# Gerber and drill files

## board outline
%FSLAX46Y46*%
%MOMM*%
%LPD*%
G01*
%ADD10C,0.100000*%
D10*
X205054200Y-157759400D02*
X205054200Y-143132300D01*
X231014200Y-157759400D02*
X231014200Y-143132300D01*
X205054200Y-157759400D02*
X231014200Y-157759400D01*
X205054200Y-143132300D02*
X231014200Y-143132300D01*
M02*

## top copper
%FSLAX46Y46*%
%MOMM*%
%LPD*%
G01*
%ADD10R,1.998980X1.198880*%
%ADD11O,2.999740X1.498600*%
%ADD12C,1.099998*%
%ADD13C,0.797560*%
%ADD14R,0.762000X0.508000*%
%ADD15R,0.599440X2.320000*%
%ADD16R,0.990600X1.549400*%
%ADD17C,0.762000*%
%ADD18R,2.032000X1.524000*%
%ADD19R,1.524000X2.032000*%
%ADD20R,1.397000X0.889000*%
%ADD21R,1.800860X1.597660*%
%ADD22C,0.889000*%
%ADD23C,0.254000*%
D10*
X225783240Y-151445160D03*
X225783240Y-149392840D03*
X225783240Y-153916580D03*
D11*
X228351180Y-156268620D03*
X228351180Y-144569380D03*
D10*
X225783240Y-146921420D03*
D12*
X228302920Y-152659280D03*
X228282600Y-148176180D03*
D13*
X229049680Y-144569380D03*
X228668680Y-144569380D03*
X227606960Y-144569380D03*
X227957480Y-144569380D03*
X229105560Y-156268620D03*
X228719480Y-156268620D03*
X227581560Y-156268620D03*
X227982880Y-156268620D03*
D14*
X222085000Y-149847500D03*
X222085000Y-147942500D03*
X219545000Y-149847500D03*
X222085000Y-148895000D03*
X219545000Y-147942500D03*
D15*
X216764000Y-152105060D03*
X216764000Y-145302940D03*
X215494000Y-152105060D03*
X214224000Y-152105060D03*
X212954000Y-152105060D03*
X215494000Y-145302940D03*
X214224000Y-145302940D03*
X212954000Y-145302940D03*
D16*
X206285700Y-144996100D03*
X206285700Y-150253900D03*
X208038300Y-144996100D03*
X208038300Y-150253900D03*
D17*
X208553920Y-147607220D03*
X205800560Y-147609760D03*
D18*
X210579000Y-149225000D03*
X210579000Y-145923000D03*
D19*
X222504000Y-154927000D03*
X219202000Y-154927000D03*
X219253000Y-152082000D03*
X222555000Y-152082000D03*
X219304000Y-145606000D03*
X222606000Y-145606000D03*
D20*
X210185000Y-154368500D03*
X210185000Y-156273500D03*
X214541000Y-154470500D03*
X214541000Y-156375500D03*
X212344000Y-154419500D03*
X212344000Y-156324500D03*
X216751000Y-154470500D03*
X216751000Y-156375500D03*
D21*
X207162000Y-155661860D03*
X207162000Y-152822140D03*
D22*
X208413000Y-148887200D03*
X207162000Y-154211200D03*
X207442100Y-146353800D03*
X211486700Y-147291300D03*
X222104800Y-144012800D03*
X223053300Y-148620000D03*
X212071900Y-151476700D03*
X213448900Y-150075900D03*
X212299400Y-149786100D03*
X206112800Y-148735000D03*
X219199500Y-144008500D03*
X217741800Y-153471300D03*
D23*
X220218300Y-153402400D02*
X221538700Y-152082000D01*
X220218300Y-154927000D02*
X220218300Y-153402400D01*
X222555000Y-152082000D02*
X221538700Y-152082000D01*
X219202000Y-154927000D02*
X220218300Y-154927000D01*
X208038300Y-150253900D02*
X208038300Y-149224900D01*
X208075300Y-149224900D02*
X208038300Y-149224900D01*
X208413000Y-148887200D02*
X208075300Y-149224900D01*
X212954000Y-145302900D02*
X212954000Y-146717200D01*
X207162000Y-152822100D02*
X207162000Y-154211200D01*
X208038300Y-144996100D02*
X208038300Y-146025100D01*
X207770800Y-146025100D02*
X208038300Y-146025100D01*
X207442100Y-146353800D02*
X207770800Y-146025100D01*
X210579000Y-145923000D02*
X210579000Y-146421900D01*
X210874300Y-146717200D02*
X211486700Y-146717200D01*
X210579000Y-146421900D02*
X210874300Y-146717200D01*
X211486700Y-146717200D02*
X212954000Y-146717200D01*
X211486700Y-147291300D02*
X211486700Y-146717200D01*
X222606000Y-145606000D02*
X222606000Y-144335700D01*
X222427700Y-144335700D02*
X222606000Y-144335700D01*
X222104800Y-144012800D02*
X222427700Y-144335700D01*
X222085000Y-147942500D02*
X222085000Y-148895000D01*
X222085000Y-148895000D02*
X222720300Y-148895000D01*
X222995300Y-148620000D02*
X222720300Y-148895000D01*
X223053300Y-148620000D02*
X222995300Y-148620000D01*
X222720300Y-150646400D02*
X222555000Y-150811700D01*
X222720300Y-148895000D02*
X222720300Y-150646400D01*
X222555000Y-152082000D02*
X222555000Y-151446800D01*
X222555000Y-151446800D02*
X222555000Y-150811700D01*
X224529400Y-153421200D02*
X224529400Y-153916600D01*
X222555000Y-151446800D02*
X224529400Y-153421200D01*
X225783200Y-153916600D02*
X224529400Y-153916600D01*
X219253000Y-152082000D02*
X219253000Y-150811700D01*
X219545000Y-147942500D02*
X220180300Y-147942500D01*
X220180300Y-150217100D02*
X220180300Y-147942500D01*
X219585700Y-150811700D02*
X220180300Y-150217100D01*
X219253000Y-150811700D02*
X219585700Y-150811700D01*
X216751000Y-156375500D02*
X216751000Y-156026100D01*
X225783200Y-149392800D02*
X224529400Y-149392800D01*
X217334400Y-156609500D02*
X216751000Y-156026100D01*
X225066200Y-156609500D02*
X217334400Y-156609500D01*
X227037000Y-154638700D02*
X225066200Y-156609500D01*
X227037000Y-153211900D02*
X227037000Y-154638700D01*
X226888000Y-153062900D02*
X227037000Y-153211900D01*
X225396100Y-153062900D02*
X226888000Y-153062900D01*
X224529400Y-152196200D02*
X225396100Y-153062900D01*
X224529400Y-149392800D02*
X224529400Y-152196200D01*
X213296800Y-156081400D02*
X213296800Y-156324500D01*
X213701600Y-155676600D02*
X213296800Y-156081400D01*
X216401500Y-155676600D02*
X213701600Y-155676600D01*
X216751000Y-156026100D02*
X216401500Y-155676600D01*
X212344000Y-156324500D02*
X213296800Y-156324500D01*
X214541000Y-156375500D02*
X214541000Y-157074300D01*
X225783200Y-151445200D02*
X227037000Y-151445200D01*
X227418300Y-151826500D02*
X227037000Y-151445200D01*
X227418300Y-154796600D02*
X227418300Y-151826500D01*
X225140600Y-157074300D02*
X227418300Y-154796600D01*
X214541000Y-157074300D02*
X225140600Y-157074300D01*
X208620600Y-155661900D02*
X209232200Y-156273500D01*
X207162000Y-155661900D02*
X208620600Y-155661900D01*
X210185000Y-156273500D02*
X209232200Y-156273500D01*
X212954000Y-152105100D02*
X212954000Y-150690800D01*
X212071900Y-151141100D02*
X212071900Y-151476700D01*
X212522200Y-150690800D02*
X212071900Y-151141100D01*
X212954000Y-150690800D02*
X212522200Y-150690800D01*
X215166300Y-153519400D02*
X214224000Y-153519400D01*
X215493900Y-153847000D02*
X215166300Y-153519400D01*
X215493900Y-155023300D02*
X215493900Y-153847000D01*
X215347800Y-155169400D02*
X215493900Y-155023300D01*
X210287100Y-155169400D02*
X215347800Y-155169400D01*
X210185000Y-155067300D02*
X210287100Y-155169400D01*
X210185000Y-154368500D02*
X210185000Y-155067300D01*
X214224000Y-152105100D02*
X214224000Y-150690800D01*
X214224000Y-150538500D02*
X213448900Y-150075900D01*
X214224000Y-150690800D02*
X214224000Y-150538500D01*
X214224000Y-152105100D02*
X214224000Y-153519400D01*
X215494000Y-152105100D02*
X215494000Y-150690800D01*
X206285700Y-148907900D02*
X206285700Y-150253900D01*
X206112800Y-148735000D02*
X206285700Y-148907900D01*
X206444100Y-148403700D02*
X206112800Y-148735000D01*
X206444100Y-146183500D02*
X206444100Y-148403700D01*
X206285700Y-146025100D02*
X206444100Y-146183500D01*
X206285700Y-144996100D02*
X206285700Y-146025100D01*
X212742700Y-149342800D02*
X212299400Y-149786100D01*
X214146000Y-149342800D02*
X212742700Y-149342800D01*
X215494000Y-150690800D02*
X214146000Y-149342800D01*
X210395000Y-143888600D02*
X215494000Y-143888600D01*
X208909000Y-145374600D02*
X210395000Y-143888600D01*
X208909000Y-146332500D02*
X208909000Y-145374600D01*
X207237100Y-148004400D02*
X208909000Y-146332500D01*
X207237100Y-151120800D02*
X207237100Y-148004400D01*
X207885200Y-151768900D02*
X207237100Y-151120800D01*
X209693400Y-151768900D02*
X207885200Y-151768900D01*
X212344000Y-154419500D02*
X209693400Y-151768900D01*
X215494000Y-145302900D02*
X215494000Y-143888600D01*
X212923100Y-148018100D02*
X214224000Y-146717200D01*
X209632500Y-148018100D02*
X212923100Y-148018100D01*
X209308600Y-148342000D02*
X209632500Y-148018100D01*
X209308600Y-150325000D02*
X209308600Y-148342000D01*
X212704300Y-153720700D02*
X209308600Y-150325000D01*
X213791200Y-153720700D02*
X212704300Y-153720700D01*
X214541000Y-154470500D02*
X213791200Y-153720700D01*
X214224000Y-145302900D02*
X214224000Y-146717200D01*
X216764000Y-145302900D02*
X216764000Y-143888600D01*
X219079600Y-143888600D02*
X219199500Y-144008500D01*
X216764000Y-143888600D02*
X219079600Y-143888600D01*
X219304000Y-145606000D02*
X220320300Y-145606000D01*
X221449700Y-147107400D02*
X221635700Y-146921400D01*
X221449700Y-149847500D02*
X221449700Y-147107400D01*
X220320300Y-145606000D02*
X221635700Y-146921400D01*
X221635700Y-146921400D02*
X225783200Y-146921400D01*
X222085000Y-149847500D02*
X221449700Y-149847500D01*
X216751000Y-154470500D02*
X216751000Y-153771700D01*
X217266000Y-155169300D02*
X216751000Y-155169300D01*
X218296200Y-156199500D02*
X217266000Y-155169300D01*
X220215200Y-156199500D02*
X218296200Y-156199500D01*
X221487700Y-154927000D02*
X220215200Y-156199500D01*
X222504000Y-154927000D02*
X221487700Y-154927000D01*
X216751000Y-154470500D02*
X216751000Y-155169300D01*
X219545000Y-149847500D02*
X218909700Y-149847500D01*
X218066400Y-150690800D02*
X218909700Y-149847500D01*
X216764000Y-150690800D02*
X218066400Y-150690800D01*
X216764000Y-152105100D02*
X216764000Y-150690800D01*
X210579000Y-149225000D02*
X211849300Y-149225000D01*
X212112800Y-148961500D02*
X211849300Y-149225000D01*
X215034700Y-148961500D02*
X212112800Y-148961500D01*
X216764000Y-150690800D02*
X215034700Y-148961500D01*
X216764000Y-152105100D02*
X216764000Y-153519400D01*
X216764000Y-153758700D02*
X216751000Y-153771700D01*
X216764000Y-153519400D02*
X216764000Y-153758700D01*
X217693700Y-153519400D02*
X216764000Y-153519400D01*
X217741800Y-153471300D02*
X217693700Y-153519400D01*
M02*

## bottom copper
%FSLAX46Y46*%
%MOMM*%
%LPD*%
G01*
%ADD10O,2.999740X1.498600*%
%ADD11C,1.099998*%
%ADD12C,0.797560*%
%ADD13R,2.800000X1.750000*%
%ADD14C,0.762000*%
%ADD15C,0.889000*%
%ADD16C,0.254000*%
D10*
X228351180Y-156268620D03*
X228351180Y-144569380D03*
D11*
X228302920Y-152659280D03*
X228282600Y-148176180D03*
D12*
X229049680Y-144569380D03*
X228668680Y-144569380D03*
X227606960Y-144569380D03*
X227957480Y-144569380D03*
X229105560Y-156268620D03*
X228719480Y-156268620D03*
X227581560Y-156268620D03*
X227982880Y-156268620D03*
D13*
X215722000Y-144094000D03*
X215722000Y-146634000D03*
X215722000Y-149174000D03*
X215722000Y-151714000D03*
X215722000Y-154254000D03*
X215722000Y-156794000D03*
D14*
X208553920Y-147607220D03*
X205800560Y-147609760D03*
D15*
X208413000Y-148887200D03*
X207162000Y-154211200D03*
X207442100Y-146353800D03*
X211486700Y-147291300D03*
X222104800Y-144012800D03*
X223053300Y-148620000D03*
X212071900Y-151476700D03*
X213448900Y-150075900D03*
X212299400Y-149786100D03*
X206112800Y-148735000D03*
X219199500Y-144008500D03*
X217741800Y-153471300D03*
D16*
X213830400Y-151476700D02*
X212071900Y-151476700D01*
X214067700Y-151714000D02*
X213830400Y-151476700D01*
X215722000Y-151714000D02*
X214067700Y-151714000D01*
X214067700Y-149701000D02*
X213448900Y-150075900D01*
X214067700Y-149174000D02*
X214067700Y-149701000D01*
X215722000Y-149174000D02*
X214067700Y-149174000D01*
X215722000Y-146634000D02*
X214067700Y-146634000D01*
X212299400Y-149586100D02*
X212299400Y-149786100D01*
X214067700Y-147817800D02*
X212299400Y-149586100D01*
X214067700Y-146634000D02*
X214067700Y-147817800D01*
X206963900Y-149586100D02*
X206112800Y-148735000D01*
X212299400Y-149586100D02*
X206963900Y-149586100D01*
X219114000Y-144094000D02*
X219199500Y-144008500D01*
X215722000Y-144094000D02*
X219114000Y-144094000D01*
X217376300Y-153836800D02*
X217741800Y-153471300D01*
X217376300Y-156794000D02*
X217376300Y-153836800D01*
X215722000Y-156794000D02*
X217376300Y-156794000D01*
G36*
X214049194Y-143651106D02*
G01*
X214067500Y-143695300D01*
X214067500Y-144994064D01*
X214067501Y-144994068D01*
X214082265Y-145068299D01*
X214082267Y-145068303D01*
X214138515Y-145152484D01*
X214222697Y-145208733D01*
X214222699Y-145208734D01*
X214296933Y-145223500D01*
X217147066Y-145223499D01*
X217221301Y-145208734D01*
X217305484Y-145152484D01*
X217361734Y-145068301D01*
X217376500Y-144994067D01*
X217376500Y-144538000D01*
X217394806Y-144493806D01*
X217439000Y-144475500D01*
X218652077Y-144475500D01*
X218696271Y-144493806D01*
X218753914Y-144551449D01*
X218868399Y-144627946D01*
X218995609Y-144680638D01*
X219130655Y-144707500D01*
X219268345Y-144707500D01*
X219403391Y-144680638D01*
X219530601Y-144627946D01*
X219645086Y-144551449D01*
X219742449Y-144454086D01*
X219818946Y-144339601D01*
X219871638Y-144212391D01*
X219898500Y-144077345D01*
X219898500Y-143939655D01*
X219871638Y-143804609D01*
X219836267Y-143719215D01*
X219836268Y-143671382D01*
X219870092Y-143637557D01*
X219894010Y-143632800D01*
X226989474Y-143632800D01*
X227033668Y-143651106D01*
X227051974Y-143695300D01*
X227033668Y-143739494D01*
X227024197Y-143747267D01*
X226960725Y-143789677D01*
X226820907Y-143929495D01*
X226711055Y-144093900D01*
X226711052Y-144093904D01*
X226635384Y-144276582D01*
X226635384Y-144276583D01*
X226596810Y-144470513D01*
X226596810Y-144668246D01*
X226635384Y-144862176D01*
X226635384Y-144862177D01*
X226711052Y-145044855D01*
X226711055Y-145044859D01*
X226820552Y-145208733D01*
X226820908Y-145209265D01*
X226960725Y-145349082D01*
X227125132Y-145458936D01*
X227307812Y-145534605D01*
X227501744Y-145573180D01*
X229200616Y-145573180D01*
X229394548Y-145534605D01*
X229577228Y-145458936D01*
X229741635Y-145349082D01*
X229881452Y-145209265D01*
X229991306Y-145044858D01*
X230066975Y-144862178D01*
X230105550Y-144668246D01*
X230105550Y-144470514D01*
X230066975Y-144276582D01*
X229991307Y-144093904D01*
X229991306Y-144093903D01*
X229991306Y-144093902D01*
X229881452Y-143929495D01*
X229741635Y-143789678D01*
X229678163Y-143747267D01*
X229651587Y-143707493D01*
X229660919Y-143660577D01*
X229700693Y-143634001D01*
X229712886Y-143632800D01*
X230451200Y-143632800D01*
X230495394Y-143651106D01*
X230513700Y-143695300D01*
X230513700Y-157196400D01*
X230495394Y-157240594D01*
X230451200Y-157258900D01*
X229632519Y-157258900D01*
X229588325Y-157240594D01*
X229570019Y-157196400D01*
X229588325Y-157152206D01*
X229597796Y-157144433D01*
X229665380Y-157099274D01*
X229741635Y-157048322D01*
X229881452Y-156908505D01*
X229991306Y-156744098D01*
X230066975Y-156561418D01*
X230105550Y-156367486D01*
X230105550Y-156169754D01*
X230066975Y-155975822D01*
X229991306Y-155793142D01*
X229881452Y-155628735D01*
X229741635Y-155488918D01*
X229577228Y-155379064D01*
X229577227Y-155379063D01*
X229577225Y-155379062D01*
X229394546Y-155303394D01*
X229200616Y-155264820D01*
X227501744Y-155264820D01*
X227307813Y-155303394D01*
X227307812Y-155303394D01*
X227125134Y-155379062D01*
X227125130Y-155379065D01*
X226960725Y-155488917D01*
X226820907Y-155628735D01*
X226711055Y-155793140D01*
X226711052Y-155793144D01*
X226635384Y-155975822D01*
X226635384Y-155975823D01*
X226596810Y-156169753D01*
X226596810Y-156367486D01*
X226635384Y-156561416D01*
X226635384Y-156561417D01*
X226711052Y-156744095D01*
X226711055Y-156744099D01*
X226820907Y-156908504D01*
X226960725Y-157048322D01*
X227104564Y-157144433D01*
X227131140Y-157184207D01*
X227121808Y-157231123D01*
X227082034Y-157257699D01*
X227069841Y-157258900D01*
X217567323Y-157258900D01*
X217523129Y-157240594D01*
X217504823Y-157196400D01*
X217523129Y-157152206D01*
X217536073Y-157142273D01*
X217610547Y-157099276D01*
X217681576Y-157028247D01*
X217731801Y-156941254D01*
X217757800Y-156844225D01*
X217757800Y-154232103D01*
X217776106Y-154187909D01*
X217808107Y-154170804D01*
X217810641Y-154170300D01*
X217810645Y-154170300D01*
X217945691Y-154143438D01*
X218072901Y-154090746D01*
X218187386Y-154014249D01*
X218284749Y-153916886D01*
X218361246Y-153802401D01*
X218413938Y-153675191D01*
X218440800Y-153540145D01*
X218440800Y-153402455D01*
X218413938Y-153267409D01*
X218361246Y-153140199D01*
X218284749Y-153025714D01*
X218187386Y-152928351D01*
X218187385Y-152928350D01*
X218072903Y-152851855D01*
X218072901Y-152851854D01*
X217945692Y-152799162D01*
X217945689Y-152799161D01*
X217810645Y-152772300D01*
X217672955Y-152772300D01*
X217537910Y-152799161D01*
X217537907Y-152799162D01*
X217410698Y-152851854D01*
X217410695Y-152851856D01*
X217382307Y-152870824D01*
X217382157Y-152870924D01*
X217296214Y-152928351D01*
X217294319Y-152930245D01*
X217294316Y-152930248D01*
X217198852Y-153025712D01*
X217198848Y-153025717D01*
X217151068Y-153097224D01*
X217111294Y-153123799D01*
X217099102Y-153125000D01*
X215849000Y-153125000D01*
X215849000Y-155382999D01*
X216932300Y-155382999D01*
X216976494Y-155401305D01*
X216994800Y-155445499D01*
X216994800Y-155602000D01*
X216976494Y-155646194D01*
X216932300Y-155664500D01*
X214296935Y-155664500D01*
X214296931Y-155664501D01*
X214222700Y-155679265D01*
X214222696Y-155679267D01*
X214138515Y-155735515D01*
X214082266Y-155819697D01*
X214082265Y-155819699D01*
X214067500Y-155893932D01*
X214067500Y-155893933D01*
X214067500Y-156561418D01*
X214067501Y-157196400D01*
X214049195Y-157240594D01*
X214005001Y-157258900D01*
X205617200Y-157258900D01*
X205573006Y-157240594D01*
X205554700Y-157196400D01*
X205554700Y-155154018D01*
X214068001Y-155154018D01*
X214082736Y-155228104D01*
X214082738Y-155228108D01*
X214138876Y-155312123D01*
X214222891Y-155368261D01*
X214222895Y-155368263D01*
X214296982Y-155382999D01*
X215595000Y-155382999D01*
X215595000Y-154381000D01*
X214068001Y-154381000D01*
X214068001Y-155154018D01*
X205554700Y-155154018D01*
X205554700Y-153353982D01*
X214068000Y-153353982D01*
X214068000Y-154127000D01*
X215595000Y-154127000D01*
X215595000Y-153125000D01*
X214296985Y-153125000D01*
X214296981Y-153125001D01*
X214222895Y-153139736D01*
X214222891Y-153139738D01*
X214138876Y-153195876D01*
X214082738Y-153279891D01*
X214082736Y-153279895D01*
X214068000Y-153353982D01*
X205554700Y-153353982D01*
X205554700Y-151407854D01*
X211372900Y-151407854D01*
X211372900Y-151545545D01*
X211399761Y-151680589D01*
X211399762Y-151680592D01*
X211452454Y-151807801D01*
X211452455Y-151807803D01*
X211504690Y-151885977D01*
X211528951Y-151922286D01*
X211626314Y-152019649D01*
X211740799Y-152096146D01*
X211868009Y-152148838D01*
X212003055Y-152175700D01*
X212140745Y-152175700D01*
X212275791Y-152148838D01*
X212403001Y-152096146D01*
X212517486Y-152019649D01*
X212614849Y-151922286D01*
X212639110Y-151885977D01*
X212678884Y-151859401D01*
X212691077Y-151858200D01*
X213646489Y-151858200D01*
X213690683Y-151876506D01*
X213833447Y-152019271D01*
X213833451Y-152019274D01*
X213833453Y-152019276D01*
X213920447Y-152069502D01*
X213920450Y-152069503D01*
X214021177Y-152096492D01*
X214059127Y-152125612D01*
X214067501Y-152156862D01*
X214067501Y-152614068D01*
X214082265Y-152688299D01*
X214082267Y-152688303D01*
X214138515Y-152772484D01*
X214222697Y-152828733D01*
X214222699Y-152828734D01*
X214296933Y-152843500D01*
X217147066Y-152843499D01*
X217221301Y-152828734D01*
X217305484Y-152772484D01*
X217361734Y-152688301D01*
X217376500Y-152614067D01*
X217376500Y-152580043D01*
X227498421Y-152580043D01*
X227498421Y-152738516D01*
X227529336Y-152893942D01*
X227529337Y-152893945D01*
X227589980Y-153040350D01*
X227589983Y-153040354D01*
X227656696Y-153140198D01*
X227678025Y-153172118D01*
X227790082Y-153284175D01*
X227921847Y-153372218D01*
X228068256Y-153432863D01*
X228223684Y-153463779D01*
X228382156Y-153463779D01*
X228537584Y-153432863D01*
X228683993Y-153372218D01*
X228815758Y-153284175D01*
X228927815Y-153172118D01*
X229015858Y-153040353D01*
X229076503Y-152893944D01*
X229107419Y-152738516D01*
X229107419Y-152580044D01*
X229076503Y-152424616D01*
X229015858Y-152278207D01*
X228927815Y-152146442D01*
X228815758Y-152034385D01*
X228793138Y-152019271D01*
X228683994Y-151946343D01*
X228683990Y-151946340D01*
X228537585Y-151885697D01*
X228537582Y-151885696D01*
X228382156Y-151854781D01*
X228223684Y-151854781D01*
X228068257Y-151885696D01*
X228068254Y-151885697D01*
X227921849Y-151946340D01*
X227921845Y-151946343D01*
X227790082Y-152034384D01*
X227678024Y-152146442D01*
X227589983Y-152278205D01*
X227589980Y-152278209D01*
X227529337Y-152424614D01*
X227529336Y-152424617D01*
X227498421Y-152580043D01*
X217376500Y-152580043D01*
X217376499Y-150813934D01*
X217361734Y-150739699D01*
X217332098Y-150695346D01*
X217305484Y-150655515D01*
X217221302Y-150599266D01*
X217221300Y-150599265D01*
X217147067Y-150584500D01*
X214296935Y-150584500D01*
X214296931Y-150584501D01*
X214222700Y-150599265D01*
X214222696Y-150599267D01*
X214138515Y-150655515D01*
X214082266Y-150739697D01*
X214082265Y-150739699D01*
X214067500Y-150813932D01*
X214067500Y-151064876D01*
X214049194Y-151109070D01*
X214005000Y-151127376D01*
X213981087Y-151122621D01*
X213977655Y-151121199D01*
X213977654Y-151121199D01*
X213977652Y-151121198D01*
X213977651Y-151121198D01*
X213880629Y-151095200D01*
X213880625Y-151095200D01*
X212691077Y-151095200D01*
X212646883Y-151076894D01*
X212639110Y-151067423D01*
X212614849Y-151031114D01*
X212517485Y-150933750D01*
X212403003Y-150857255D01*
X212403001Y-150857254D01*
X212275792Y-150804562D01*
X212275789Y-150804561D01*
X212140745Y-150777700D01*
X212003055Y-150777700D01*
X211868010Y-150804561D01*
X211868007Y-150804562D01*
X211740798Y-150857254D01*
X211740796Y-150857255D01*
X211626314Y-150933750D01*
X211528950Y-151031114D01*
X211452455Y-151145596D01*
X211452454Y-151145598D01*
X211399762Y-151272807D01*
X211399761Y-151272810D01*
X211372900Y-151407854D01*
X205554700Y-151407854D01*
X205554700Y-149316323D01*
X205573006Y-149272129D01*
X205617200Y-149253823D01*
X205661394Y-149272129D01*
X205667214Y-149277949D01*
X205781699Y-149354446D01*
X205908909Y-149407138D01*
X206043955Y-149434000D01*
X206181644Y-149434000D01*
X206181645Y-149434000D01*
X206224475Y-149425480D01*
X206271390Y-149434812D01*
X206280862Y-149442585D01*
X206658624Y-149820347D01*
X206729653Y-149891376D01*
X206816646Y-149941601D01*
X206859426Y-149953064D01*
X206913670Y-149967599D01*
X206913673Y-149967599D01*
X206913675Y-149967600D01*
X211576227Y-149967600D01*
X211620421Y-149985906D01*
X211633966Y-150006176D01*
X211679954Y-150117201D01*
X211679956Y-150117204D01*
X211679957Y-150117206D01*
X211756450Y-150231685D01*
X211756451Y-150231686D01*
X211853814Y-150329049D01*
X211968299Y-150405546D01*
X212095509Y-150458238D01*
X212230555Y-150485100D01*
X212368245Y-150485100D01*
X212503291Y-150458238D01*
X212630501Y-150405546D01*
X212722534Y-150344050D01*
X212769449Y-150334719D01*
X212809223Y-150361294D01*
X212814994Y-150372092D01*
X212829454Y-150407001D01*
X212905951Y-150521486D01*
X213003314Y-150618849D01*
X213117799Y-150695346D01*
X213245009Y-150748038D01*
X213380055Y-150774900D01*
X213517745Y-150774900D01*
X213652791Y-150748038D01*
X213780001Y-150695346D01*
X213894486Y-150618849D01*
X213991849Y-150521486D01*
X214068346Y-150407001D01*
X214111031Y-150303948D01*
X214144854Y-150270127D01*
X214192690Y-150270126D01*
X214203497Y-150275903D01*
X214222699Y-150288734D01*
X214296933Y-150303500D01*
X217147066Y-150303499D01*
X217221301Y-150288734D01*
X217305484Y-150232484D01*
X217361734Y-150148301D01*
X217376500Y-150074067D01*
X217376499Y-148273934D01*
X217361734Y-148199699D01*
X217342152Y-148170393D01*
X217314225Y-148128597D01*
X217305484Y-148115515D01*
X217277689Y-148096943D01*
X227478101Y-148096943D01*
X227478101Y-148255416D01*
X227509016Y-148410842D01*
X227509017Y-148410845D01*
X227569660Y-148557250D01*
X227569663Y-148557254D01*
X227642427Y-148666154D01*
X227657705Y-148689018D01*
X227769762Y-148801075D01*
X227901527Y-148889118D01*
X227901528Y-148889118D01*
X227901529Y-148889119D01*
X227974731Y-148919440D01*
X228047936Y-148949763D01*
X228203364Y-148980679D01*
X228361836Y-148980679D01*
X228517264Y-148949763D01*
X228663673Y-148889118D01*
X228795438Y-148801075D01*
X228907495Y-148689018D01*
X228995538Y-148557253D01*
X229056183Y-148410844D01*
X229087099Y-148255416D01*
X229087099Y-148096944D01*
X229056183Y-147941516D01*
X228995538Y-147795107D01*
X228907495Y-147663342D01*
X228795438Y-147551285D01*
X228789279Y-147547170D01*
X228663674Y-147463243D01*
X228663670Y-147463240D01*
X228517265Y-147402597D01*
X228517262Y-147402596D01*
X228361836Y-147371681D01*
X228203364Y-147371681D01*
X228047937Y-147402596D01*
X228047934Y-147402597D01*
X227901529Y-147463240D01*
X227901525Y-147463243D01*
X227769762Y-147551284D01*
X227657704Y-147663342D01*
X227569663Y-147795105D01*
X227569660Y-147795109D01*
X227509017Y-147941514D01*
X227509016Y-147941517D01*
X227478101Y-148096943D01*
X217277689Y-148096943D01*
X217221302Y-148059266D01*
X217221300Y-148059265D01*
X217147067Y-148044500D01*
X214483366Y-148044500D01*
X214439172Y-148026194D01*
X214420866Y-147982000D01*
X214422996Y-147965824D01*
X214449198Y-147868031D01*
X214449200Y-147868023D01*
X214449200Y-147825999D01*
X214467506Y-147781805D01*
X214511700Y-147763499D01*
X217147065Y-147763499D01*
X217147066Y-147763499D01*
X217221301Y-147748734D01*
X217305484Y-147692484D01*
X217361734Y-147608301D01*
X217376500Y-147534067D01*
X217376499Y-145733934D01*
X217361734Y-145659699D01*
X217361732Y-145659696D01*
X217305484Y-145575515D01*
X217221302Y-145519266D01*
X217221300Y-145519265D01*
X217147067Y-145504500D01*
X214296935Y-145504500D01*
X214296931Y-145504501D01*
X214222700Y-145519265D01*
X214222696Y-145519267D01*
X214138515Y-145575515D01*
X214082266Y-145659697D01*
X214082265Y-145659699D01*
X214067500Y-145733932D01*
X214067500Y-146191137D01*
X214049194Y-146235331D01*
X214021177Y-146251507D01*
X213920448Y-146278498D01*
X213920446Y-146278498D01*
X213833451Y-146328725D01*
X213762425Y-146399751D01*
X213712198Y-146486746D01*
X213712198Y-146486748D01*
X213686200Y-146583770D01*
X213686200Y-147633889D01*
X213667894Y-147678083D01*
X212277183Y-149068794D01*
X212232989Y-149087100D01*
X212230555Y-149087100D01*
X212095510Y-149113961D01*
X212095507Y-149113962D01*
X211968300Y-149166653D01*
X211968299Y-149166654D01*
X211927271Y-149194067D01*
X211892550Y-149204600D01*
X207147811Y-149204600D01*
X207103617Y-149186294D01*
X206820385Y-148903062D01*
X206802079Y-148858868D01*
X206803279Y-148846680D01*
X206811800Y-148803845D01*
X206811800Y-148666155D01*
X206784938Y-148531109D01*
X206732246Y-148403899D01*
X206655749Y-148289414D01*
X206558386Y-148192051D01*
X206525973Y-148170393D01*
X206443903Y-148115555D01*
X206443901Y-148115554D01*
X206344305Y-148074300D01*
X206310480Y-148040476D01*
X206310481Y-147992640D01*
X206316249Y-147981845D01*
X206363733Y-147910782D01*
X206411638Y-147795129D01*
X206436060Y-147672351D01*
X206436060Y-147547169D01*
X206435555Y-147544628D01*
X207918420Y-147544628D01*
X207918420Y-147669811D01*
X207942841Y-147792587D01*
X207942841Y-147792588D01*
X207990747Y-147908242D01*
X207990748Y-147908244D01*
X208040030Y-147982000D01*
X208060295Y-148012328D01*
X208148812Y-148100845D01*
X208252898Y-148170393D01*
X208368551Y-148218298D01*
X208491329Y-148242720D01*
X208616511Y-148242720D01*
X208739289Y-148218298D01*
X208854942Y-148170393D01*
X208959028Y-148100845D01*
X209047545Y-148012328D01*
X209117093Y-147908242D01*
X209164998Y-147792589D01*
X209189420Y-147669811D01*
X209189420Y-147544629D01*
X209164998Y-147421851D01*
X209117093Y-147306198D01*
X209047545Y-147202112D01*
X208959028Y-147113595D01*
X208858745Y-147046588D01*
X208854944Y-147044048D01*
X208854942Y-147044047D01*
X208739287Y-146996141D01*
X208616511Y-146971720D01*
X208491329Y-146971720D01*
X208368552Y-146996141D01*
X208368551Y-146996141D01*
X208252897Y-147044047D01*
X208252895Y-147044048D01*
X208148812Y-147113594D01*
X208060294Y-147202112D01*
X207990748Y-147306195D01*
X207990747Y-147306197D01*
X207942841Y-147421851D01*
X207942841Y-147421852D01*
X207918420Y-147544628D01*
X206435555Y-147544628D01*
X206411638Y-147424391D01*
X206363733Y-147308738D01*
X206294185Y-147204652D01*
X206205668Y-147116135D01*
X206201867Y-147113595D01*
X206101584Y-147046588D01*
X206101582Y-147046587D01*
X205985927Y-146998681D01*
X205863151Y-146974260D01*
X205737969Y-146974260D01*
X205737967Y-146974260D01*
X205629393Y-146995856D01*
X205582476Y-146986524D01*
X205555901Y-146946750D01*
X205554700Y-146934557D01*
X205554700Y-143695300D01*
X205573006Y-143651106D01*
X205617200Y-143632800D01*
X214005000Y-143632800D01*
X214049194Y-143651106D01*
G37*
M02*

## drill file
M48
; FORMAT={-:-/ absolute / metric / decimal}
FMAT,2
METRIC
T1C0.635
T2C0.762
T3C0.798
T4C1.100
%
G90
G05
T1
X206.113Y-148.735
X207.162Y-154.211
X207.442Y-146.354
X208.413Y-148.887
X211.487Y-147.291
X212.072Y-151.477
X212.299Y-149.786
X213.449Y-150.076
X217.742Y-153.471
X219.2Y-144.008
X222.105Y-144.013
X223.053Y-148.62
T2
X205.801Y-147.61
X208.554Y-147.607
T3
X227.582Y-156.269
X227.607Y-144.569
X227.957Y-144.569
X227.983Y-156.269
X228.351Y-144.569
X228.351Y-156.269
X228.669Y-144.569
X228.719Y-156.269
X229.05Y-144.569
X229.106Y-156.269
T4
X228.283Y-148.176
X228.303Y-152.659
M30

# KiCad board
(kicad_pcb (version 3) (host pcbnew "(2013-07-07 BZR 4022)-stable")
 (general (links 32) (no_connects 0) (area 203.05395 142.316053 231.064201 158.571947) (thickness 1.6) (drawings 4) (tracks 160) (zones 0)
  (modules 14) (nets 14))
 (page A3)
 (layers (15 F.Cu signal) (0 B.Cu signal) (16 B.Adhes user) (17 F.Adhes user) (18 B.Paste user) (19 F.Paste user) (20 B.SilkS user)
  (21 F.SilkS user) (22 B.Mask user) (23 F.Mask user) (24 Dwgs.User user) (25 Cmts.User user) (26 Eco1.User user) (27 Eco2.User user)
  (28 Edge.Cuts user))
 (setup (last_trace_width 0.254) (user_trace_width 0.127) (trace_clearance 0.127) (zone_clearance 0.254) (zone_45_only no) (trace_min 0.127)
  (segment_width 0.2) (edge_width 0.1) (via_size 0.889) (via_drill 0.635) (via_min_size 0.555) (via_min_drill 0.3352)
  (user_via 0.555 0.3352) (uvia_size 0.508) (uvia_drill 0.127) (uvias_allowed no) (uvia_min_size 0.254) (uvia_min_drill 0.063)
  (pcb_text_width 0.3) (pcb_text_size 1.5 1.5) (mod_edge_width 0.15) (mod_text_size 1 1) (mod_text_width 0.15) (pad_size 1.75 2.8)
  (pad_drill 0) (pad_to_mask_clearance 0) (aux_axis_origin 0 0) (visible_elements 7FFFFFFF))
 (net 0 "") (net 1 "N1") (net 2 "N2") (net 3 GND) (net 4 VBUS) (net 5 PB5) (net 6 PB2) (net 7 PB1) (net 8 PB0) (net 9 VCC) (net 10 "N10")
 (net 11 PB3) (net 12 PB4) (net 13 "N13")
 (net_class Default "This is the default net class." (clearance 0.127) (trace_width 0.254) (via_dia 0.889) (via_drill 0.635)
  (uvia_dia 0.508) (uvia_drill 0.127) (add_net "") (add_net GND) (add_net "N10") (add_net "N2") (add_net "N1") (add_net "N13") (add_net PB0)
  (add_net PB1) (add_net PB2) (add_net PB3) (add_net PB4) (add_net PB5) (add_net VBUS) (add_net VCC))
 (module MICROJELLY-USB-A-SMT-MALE (layer F.Cu) (at 229.451 150.419 270)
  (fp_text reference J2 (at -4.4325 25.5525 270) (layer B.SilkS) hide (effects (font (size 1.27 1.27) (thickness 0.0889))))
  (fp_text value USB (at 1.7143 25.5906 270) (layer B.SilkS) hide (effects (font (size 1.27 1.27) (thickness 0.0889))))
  (pad 2 smd rect (at 1.02616 3.66776 270) (size 1.19888 1.99898) (layers F.Cu F.Paste F.Mask) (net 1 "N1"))
  (pad 3 smd rect (at -1.02616 3.66776 270) (size 1.19888 1.99898) (layers F.Cu F.Paste F.Mask) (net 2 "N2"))
  (pad 1 smd rect (at 3.49758 3.66776 270) (size 1.19888 1.99898) (layers F.Cu F.Paste F.Mask) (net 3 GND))
  (pad P$1 thru_hole oval (at 5.84962 1.09982 270) (size 1.4986 2.99974) (drill 0.79756) (layers *.Cu *.Mask F.Paste F.SilkS))
  (pad P$3 thru_hole oval (at -5.84962 1.09982 270) (size 1.4986 2.99974) (drill 0.79756) (layers *.Cu *.Mask F.Paste F.SilkS))
  (pad 4 smd rect (at -3.49758 3.66776 270) (size 1.19888 1.99898) (layers F.Cu F.Paste F.Mask) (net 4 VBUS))
  (pad P$4 thru_hole circle (at 2.24028 1.14808 270) (size 1.099998 1.099998) (drill 1.099998) (layers *.Cu *.Mask F.SilkS))
  (pad P$5 thru_hole circle (at -2.24282 1.1684 270) (size 1.099998 1.099998) (drill 1.099998) (layers *.Cu *.Mask F.SilkS))
  (pad P$4 thru_hole circle (at -5.84962 0.40132 270) (size 0.79756 0.79756) (drill 0.79756) (layers *.Cu F.Paste F.SilkS F.Mask))
  (pad P$5 thru_hole circle (at -5.84962 0.78232 270) (size 0.79756 0.79756) (drill 0.79756) (layers *.Cu F.Paste F.SilkS F.Mask))
  (pad P$6 thru_hole circle (at -5.84962 1.84404 270) (size 0.79756 0.79756) (drill 0.79756) (layers *.Cu F.Paste F.SilkS F.Mask))
  (pad P$7 thru_hole circle (at -5.84962 1.49352 270) (size 0.79756 0.79756) (drill 0.79756) (layers *.Cu F.Paste F.SilkS F.Mask))
  (pad P$2 thru_hole circle (at 5.84962 0.34544 270) (size 0.79756 0.79756) (drill 0.79756) (layers *.Cu F.Paste F.SilkS F.Mask))
  (pad P$3 thru_hole circle (at 5.84962 0.73152 270) (size 0.79756 0.79756) (drill 0.79756) (layers *.Cu F.Paste F.SilkS F.Mask))
  (pad P$4 thru_hole circle (at 5.84962 1.86944 270) (size 0.79756 0.79756) (drill 0.79756) (layers *.Cu F.Paste F.SilkS F.Mask))
  (pad P$5 thru_hole circle (at 5.84962 1.46812 270) (size 0.79756 0.79756) (drill 0.79756) (layers *.Cu F.Paste F.SilkS F.Mask)))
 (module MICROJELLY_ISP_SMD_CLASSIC (layer B.Cu) (at 213.944 150.444 270)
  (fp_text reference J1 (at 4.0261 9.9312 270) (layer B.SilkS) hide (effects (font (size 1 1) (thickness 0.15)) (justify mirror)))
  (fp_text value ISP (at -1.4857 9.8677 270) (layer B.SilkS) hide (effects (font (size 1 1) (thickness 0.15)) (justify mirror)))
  (pad 5 smd rect (at -6.35 -1.778 270) (size 1.75 2.8) (layers B.Cu B.Paste B.Mask) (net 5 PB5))
  (pad 3 smd rect (at -3.81 -1.778 270) (size 1.75 2.8) (layers B.Cu B.Paste B.Mask) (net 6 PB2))
  (pad 1 smd rect (at -1.27 -1.778 270) (size 1.75 2.8) (layers B.Cu B.Paste B.Mask) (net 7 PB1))
  (pad 4 smd rect (at 1.27 -1.778 270) (size 1.75 2.8) (layers B.Cu B.Paste B.Mask) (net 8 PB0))
  (pad 6 smd rect (at 3.81 -1.778 270) (size 1.75 2.8) (layers B.Cu B.Paste B.Mask) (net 3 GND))
  (pad 2 smd rect (at 6.35 -1.778 270) (size 1.75 2.8) (layers B.Cu B.Paste B.Mask) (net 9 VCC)))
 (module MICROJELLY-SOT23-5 (layer F.Cu) (at 220.815 148.895 90)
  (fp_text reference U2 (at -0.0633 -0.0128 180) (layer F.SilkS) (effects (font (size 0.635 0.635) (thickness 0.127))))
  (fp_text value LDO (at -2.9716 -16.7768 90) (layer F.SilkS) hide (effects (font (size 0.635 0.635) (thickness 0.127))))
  (pad 1 smd rect (at -0.9525 1.27 90) (size 0.508 0.762) (layers F.Cu F.Paste F.Mask) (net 4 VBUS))
  (pad 3 smd rect (at 0.9525 1.27 90) (size 0.508 0.762) (layers F.Cu F.Paste F.Mask) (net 3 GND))
  (pad 5 smd rect (at -0.9525 -1.27 90) (size 0.508 0.762) (layers F.Cu F.Paste F.Mask) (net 9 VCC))
  (pad 2 smd rect (at 0 1.27 90) (size 0.508 0.762) (layers F.Cu F.Paste F.Mask) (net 3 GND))
  (pad 4 smd rect (at 0.9525 -1.27 90) (size 0.508 0.762) (layers F.Cu F.Paste F.Mask) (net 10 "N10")))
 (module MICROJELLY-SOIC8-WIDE (layer F.Cu) (at 214.859 148.704 180)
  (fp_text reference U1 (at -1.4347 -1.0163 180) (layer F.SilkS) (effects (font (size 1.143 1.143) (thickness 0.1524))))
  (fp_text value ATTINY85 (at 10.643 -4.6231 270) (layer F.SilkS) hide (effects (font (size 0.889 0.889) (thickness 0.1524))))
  (pad 8 smd rect (at -1.905 -3.40106 180) (size 0.59944 2.32) (layers F.Cu F.Paste F.Mask) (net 9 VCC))
  (pad 1 smd rect (at -1.905 3.40106 180) (size 0.59944 2.32) (layers F.Cu F.Paste F.Mask) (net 5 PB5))
  (pad 7 smd rect (at -0.635 -3.40106 180) (size 0.59944 2.32) (layers F.Cu F.Paste F.Mask) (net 6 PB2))
  (pad 6 smd rect (at 0.635 -3.40106 180) (size 0.59944 2.32) (layers F.Cu F.Paste F.Mask) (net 7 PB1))
  (pad 5 smd rect (at 1.905 -3.40106 180) (size 0.59944 2.32) (layers F.Cu F.Paste F.Mask) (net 8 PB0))
  (pad 2 smd rect (at -0.635 3.40106 180) (size 0.59944 2.32) (layers F.Cu F.Paste F.Mask) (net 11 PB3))
  (pad 3 smd rect (at 0.635 3.40106 180) (size 0.59944 2.32) (layers F.Cu F.Paste F.Mask) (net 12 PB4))
  (pad 4 smd rect (at 1.905 3.40106 180) (size 0.59944 2.32) (layers F.Cu F.Paste F.Mask) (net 3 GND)))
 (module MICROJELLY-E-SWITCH (layer F.Cu) (at 207.162 147.625 270)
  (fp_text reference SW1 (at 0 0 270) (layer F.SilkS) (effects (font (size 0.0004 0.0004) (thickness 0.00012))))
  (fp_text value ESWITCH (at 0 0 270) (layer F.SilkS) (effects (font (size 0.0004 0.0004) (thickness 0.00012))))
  (pad 1 smd rect (at -2.6289 0.8763 270) (size 1.5494 0.9906) (layers F.Cu F.Paste F.Mask) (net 6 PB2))
  (pad 1 smd rect (at 2.6289 0.8763 270) (size 1.5494 0.9906) (layers F.Cu F.Paste F.Mask) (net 6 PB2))
  (pad 2 smd rect (at -2.6289 -0.8763 270) (size 1.5494 0.9906) (layers F.Cu F.Paste F.Mask) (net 3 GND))
  (pad 2 smd rect (at 2.6289 -0.8763 270) (size 1.5494 0.9906) (layers F.Cu F.Paste F.Mask) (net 3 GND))
  (pad P$5 thru_hole circle (at -0.01778 -1.39192 270) (size 0.762 0.762) (drill 0.762) (layers *.Cu *.Mask F.SilkS))
  (pad P$6 thru_hole circle (at -0.01524 1.36144 270) (size 0.762 0.762) (drill 0.762) (layers *.Cu *.Mask F.SilkS)))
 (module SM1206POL (layer F.Cu) (at 210.579 147.574 90)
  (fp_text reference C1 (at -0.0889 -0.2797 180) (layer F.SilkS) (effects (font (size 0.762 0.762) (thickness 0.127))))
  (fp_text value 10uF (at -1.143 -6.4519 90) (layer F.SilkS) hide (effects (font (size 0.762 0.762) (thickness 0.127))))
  (pad 1 smd rect (at -1.651 0 90) (size 1.524 2.032) (layers F.Cu F.Paste F.Mask) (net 9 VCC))
  (pad 2 smd rect (at 1.651 0 90) (size 1.524 2.032) (layers F.Cu F.Paste F.Mask) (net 3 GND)))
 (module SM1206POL (layer F.Cu) (at 220.853 154.927 180)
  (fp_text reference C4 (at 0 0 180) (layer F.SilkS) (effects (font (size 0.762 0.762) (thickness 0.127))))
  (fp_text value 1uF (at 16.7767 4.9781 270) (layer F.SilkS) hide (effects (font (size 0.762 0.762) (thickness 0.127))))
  (pad 1 smd rect (at -1.651 0 180) (size 1.524 2.032) (layers F.Cu F.Paste F.Mask) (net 9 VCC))
  (pad 2 smd rect (at 1.651 0 180) (size 1.524 2.032) (layers F.Cu F.Paste F.Mask) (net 3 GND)))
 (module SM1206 (layer F.Cu) (at 220.904 152.082)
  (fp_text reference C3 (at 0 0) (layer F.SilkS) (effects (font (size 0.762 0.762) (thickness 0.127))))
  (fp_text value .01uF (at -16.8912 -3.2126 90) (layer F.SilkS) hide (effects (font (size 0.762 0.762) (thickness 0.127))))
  (pad 1 smd rect (at -1.651 0) (size 1.524 2.032) (layers F.Cu F.Paste F.Mask) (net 10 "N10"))
  (pad 2 smd rect (at 1.651 0) (size 1.524 2.032) (layers F.Cu F.Paste F.Mask) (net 3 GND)))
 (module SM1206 (layer F.Cu) (at 220.955 145.606)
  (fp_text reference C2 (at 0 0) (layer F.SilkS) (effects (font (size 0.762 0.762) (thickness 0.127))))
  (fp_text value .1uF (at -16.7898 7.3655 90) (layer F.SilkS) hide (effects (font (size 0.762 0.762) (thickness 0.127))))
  (pad 1 smd rect (at -1.651 0) (size 1.524 2.032) (layers F.Cu F.Paste F.Mask) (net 4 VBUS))
  (pad 2 smd rect (at 1.651 0) (size 1.524 2.032) (layers F.Cu F.Paste F.Mask) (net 3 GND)))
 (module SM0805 (layer F.Cu) (at 210.185 155.321 270)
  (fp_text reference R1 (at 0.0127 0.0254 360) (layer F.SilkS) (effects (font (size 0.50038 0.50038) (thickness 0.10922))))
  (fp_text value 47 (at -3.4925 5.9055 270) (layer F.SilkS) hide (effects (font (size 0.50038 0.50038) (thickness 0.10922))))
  (pad 1 smd rect (at -0.9525 0 270) (size 0.889 1.397) (layers F.Cu F.Paste F.Mask) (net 7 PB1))
  (pad 2 smd rect (at 0.9525 0 270) (size 0.889 1.397) (layers F.Cu F.Paste F.Mask) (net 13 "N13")))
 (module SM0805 (layer F.Cu) (at 214.541 155.423 270)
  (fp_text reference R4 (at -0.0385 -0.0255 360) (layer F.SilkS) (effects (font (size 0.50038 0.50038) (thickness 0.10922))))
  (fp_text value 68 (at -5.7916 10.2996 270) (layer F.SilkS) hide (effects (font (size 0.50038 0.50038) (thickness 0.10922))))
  (pad 1 smd rect (at -0.9525 0 270) (size 0.889 1.397) (layers F.Cu F.Paste F.Mask) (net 12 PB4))
  (pad 2 smd rect (at 0.9525 0 270) (size 0.889 1.397) (layers F.Cu F.Paste F.Mask) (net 1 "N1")))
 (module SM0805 (layer F.Cu) (at 212.344 155.372 270)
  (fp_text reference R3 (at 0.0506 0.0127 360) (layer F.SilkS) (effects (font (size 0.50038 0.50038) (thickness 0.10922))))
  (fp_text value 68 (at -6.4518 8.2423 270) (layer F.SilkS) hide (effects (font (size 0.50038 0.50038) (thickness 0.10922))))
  (pad 1 smd rect (at -0.9525 0 270) (size 0.889 1.397) (layers F.Cu F.Paste F.Mask) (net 11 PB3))
  (pad 2 smd rect (at 0.9525 0 270) (size 0.889 1.397) (layers F.Cu F.Paste F.Mask) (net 2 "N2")))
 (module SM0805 (layer F.Cu) (at 216.751 155.423 270)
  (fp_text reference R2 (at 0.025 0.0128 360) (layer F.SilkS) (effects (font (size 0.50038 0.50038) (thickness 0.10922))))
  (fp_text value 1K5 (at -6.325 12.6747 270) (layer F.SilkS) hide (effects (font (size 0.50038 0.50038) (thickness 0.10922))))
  (pad 1 smd rect (at -0.9525 0 270) (size 0.889 1.397) (layers F.Cu F.Paste F.Mask) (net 9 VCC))
  (pad 2 smd rect (at 0.9525 0 270) (size 0.889 1.397) (layers F.Cu F.Paste F.Mask) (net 2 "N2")))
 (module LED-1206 (layer F.Cu) (at 207.162 154.242 90)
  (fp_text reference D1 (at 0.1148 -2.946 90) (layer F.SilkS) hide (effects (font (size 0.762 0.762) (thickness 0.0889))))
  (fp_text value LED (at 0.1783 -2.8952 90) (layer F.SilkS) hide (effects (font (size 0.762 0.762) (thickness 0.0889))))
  (pad 1 smd rect (at -1.41986 0 90) (size 1.59766 1.80086) (layers F.Cu F.Paste F.Mask) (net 13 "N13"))
  (pad 2 smd rect (at 1.41986 0 90) (size 1.59766 1.80086) (layers F.Cu F.Paste F.Mask) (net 3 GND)))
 (gr_line (start 205.0542 157.7594) (end 205.0542 143.1323) (angle 90) (layer Edge.Cuts) (width 0.1))
 (gr_line (start 231.0142 157.7594) (end 231.0142 143.1323) (angle 90) (layer Edge.Cuts) (width 0.1))
 (gr_line (start 205.0542 157.7594) (end 231.0142 157.7594) (angle 90) (layer Edge.Cuts) (width 0.1))
 (gr_line (start 205.0542 143.1323) (end 231.0142 143.1323) (angle 90) (layer Edge.Cuts) (width 0.1))
 (via (at 208.413 148.8872) (size 0.889) (layers F.Cu B.Cu) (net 3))
 (via (at 207.162 154.2112) (size 0.889) (layers F.Cu B.Cu) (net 3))
 (via (at 207.4421 146.3538) (size 0.889) (layers F.Cu B.Cu) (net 3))
 (via (at 211.4867 147.2913) (size 0.889) (layers F.Cu B.Cu) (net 3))
 (via (at 222.1048 144.0128) (size 0.889) (layers F.Cu B.Cu) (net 3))
 (via (at 223.0533 148.62) (size 0.889) (layers F.Cu B.Cu) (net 3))
 (segment (start 220.2183 153.4024) (end 221.5387 152.082) (width 0.254) (layer F.Cu) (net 3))
 (segment (start 220.2183 154.927) (end 220.2183 153.4024) (width 0.254) (layer F.Cu) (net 3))
 (segment (start 222.555 152.082) (end 221.5387 152.082) (width 0.254) (layer F.Cu) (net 3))
 (segment (start 219.202 154.927) (end 220.2183 154.927) (width 0.254) (layer F.Cu) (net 3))
 (segment (start 208.0383 150.2539) (end 208.0383 149.2249) (width 0.254) (layer F.Cu) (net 3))
 (segment (start 208.0753 149.2249) (end 208.0383 149.2249) (width 0.254) (layer F.Cu) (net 3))
 (segment (start 208.413 148.8872) (end 208.0753 149.2249) (width 0.254) (layer F.Cu) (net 3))
 (segment (start 212.954 145.3029) (end 212.954 146.7172) (width 0.254) (layer F.Cu) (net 3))
 (segment (start 207.162 152.8221) (end 207.162 154.2112) (width 0.254) (layer F.Cu) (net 3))
 (segment (start 208.0383 144.9961) (end 208.0383 146.0251) (width 0.254) (layer F.Cu) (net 3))
 (segment (start 207.7708 146.0251) (end 208.0383 146.0251) (width 0.254) (layer F.Cu) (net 3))
 (segment (start 207.4421 146.3538) (end 207.7708 146.0251) (width 0.254) (layer F.Cu) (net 3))
 (segment (start 210.579 145.923) (end 210.579 146.4219) (width 0.254) (layer F.Cu) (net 3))
 (segment (start 210.8743 146.7172) (end 211.4867 146.7172) (width 0.254) (layer F.Cu) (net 3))
 (segment (start 210.579 146.4219) (end 210.8743 146.7172) (width 0.254) (layer F.Cu) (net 3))
 (segment (start 211.4867 146.7172) (end 212.954 146.7172) (width 0.254) (layer F.Cu) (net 3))
 (segment (start 211.4867 147.2913) (end 211.4867 146.7172) (width 0.254) (layer F.Cu) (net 3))
 (segment (start 222.606 145.606) (end 222.606 144.3357) (width 0.254) (layer F.Cu) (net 3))
 (segment (start 222.4277 144.3357) (end 222.606 144.3357) (width 0.254) (layer F.Cu) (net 3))
 (segment (start 222.1048 144.0128) (end 222.4277 144.3357) (width 0.254) (layer F.Cu) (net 3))
 (segment (start 222.085 147.9425) (end 222.085 148.895) (width 0.254) (layer F.Cu) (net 3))
 (segment (start 222.085 148.895) (end 222.7203 148.895) (width 0.254) (layer F.Cu) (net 3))
 (segment (start 222.9953 148.62) (end 222.7203 148.895) (width 0.254) (layer F.Cu) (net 3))
 (segment (start 223.0533 148.62) (end 222.9953 148.62) (width 0.254) (layer F.Cu) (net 3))
 (segment (start 222.7203 150.6464) (end 222.555 150.8117) (width 0.254) (layer F.Cu) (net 3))
 (segment (start 222.7203 148.895) (end 222.7203 150.6464) (width 0.254) (layer F.Cu) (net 3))
 (segment (start 222.555 152.082) (end 222.555 151.4468) (width 0.254) (layer F.Cu) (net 3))
 (segment (start 222.555 151.4468) (end 222.555 150.8117) (width 0.254) (layer F.Cu) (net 3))
 (segment (start 224.5294 153.4212) (end 224.5294 153.9166) (width 0.254) (layer F.Cu) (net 3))
 (segment (start 222.555 151.4468) (end 224.5294 153.4212) (width 0.254) (layer F.Cu) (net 3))
 (segment (start 225.7832 153.9166) (end 224.5294 153.9166) (width 0.254) (layer F.Cu) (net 3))
 (segment (start 219.253 152.082) (end 219.253 150.8117) (width 0.254) (layer F.Cu) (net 10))
 (segment (start 219.545 147.9425) (end 220.1803 147.9425) (width 0.254) (layer F.Cu) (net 10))
 (segment (start 220.1803 150.2171) (end 220.1803 147.9425) (width 0.254) (layer F.Cu) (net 10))
 (segment (start 219.5857 150.8117) (end 220.1803 150.2171) (width 0.254) (layer F.Cu) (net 10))
 (segment (start 219.253 150.8117) (end 219.5857 150.8117) (width 0.254) (layer F.Cu) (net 10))
 (segment (start 216.751 156.3755) (end 216.751 156.0261) (width 0.254) (layer F.Cu) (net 2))
 (segment (start 225.7832 149.3928) (end 224.5294 149.3928) (width 0.254) (layer F.Cu) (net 2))
 (segment (start 217.3344 156.6095) (end 216.751 156.0261) (width 0.254) (layer F.Cu) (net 2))
 (segment (start 225.0662 156.6095) (end 217.3344 156.6095) (width 0.254) (layer F.Cu) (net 2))
 (segment (start 227.037 154.6387) (end 225.0662 156.6095) (width 0.254) (layer F.Cu) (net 2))
 (segment (start 227.037 153.2119) (end 227.037 154.6387) (width 0.254) (layer F.Cu) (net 2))
 (segment (start 226.888 153.0629) (end 227.037 153.2119) (width 0.254) (layer F.Cu) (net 2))
 (segment (start 225.3961 153.0629) (end 226.888 153.0629) (width 0.254) (layer F.Cu) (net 2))
 (segment (start 224.5294 152.1962) (end 225.3961 153.0629) (width 0.254) (layer F.Cu) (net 2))
 (segment (start 224.5294 149.3928) (end 224.5294 152.1962) (width 0.254) (layer F.Cu) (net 2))
 (segment (start 213.2968 156.0814) (end 213.2968 156.3245) (width 0.254) (layer F.Cu) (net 2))
 (segment (start 213.7016 155.6766) (end 213.2968 156.0814) (width 0.254) (layer F.Cu) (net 2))
 (segment (start 216.4015 155.6766) (end 213.7016 155.6766) (width 0.254) (layer F.Cu) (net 2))
 (segment (start 216.751 156.0261) (end 216.4015 155.6766) (width 0.254) (layer F.Cu) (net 2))
 (segment (start 212.344 156.3245) (end 213.2968 156.3245) (width 0.254) (layer F.Cu) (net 2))
 (segment (start 214.541 156.3755) (end 214.541 157.0743) (width 0.254) (layer F.Cu) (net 1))
 (segment (start 225.7832 151.4452) (end 227.037 151.4452) (width 0.254) (layer F.Cu) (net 1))
 (segment (start 227.4183 151.8265) (end 227.037 151.4452) (width 0.254) (layer F.Cu) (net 1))
 (segment (start 227.4183 154.7966) (end 227.4183 151.8265) (width 0.254) (layer F.Cu) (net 1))
 (segment (start 225.1406 157.0743) (end 227.4183 154.7966) (width 0.254) (layer F.Cu) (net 1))
 (segment (start 214.541 157.0743) (end 225.1406 157.0743) (width 0.254) (layer F.Cu) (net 1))
 (segment (start 208.6206 155.6619) (end 209.2322 156.2735) (width 0.254) (layer F.Cu) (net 13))
 (segment (start 207.162 155.6619) (end 208.6206 155.6619) (width 0.254) (layer F.Cu) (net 13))
 (segment (start 210.185 156.2735) (end 209.2322 156.2735) (width 0.254) (layer F.Cu) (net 13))
 (via (at 212.0719 151.4767) (size 0.889) (layers F.Cu B.Cu) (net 8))
 (segment (start 212.954 152.1051) (end 212.954 150.6908) (width 0.254) (layer F.Cu) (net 8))
 (segment (start 213.8304 151.4767) (end 212.0719 151.4767) (width 0.254) (layer B.Cu) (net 8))
 (segment (start 214.0677 151.714) (end 213.8304 151.4767) (width 0.254) (layer B.Cu) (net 8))
 (segment (start 212.0719 151.1411) (end 212.0719 151.4767) (width 0.254) (layer F.Cu) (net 8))
 (segment (start 212.5222 150.6908) (end 212.0719 151.1411) (width 0.254) (layer F.Cu) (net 8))
 (segment (start 212.954 150.6908) (end 212.5222 150.6908) (width 0.254) (layer F.Cu) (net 8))
 (segment (start 215.722 151.714) (end 214.0677 151.714) (width 0.254) (layer B.Cu) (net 8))
 (via (at 213.4489 150.0759) (size 0.889) (layers F.Cu B.Cu) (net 7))
 (segment (start 215.1663 153.5194) (end 214.224 153.5194) (width 0.254) (layer F.Cu) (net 7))
 (segment (start 215.4939 153.847) (end 215.1663 153.5194) (width 0.254) (layer F.Cu) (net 7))
 (segment (start 215.4939 155.0233) (end 215.4939 153.847) (width 0.254) (layer F.Cu) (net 7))
 (segment (start 215.3478 155.1694) (end 215.4939 155.0233) (width 0.254) (layer F.Cu) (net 7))
 (segment (start 210.2871 155.1694) (end 215.3478 155.1694) (width 0.254) (layer F.Cu) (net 7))
 (segment (start 210.185 155.0673) (end 210.2871 155.1694) (width 0.254) (layer F.Cu) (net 7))
 (segment (start 210.185 154.3685) (end 210.185 155.0673) (width 0.254) (layer F.Cu) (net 7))
 (segment (start 214.224 152.1051) (end 214.224 150.6908) (width 0.254) (layer F.Cu) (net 7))
 (segment (start 214.0677 149.701) (end 213.4489 150.0759) (width 0.254) (layer B.Cu) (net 7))
 (segment (start 214.0677 149.174) (end 214.0677 149.701) (width 0.254) (layer B.Cu) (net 7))
 (segment (start 214.224 150.5385) (end 213.4489 150.0759) (width 0.254) (layer F.Cu) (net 7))
 (segment (start 214.224 150.6908) (end 214.224 150.5385) (width 0.254) (layer F.Cu) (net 7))
 (segment (start 215.722 149.174) (end 214.0677 149.174) (width 0.254) (layer B.Cu) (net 7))
 (segment (start 214.224 152.1051) (end 214.224 153.5194) (width 0.254) (layer F.Cu) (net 7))
 (via (at 212.2994 149.7861) (size 0.889) (layers F.Cu B.Cu) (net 6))
 (via (at 206.1128 148.735) (size 0.889) (layers F.Cu B.Cu) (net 6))
 (segment (start 215.494 152.1051) (end 215.494 150.6908) (width 0.254) (layer F.Cu) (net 6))
 (segment (start 215.722 146.634) (end 214.0677 146.634) (width 0.254) (layer B.Cu) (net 6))
 (segment (start 212.2994 149.5861) (end 212.2994 149.7861) (width 0.254) (layer B.Cu) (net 6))
 (segment (start 214.0677 147.8178) (end 212.2994 149.5861) (width 0.254) (layer B.Cu) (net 6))
 (segment (start 214.0677 146.634) (end 214.0677 147.8178) (width 0.254) (layer B.Cu) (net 6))
 (segment (start 206.9639 149.5861) (end 206.1128 148.735) (width 0.254) (layer B.Cu) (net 6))
 (segment (start 212.2994 149.5861) (end 206.9639 149.5861) (width 0.254) (layer B.Cu) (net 6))
 (segment (start 206.2857 148.9079) (end 206.2857 150.2539) (width 0.254) (layer F.Cu) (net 6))
 (segment (start 206.1128 148.735) (end 206.2857 148.9079) (width 0.254) (layer F.Cu) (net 6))
 (segment (start 206.4441 148.4037) (end 206.1128 148.735) (width 0.254) (layer F.Cu) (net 6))
 (segment (start 206.4441 146.1835) (end 206.4441 148.4037) (width 0.254) (layer F.Cu) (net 6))
 (segment (start 206.2857 146.0251) (end 206.4441 146.1835) (width 0.254) (layer F.Cu) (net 6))
 (segment (start 206.2857 144.9961) (end 206.2857 146.0251) (width 0.254) (layer F.Cu) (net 6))
 (segment (start 212.7427 149.3428) (end 212.2994 149.7861) (width 0.254) (layer F.Cu) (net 6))
 (segment (start 214.146 149.3428) (end 212.7427 149.3428) (width 0.254) (layer F.Cu) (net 6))
 (segment (start 215.494 150.6908) (end 214.146 149.3428) (width 0.254) (layer F.Cu) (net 6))
 (segment (start 210.395 143.8886) (end 215.494 143.8886) (width 0.254) (layer F.Cu) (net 11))
 (segment (start 208.909 145.3746) (end 210.395 143.8886) (width 0.254) (layer F.Cu) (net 11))
 (segment (start 208.909 146.3325) (end 208.909 145.3746) (width 0.254) (layer F.Cu) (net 11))
 (segment (start 207.2371 148.0044) (end 208.909 146.3325) (width 0.254) (layer F.Cu) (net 11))
 (segment (start 207.2371 151.1208) (end 207.2371 148.0044) (width 0.254) (layer F.Cu) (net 11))
 (segment (start 207.8852 151.7689) (end 207.2371 151.1208) (width 0.254) (layer F.Cu) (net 11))
 (segment (start 209.6934 151.7689) (end 207.8852 151.7689) (width 0.254) (layer F.Cu) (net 11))
 (segment (start 212.344 154.4195) (end 209.6934 151.7689) (width 0.254) (layer F.Cu) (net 11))
 (segment (start 215.494 145.3029) (end 215.494 143.8886) (width 0.254) (layer F.Cu) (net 11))
 (segment (start 212.9231 148.0181) (end 214.224 146.7172) (width 0.254) (layer F.Cu) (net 12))
 (segment (start 209.6325 148.0181) (end 212.9231 148.0181) (width 0.254) (layer F.Cu) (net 12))
 (segment (start 209.3086 148.342) (end 209.6325 148.0181) (width 0.254) (layer F.Cu) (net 12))
 (segment (start 209.3086 150.325) (end 209.3086 148.342) (width 0.254) (layer F.Cu) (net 12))
 (segment (start 212.7043 153.7207) (end 209.3086 150.325) (width 0.254) (layer F.Cu) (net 12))
 (segment (start 213.7912 153.7207) (end 212.7043 153.7207) (width 0.254) (layer F.Cu) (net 12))
 (segment (start 214.541 154.4705) (end 213.7912 153.7207) (width 0.254) (layer F.Cu) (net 12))
 (segment (start 214.224 145.3029) (end 214.224 146.7172) (width 0.254) (layer F.Cu) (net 12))
 (via (at 219.1995 144.0085) (size 0.889) (layers F.Cu B.Cu) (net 5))
 (segment (start 216.764 145.3029) (end 216.764 143.8886) (width 0.254) (layer F.Cu) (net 5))
 (segment (start 219.114 144.094) (end 219.1995 144.0085) (width 0.254) (layer B.Cu) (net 5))
 (segment (start 215.722 144.094) (end 219.114 144.094) (width 0.254) (layer B.Cu) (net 5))
 (segment (start 219.0796 143.8886) (end 219.1995 144.0085) (width 0.254) (layer F.Cu) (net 5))
 (segment (start 216.764 143.8886) (end 219.0796 143.8886) (width 0.254) (layer F.Cu) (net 5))
 (segment (start 219.304 145.606) (end 220.3203 145.606) (width 0.254) (layer F.Cu) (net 4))
 (segment (start 221.4497 147.1074) (end 221.6357 146.9214) (width 0.254) (layer F.Cu) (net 4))
 (segment (start 221.4497 149.8475) (end 221.4497 147.1074) (width 0.254) (layer F.Cu) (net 4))
 (segment (start 220.3203 145.606) (end 221.6357 146.9214) (width 0.254) (layer F.Cu) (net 4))
 (segment (start 221.6357 146.9214) (end 225.7832 146.9214) (width 0.254) (layer F.Cu) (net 4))
 (segment (start 222.085 149.8475) (end 221.4497 149.8475) (width 0.254) (layer F.Cu) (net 4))
 (via (at 217.7418 153.4713) (size 0.889) (layers F.Cu B.Cu) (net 9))
 (segment (start 216.751 154.4705) (end 216.751 153.7717) (width 0.254) (layer F.Cu) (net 9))
 (segment (start 217.266 155.1693) (end 216.751 155.1693) (width 0.254) (layer F.Cu) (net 9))
 (segment (start 218.2962 156.1995) (end 217.266 155.1693) (width 0.254) (layer F.Cu) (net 9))
 (segment (start 220.2152 156.1995) (end 218.2962 156.1995) (width 0.254) (layer F.Cu) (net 9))
 (segment (start 221.4877 154.927) (end 220.2152 156.1995) (width 0.254) (layer F.Cu) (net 9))
 (segment (start 222.504 154.927) (end 221.4877 154.927) (width 0.254) (layer F.Cu) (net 9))
 (segment (start 216.751 154.4705) (end 216.751 155.1693) (width 0.254) (layer F.Cu) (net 9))
 (segment (start 219.545 149.8475) (end 218.9097 149.8475) (width 0.254) (layer F.Cu) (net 9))
 (segment (start 218.0664 150.6908) (end 218.9097 149.8475) (width 0.254) (layer F.Cu) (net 9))
 (segment (start 216.764 150.6908) (end 218.0664 150.6908) (width 0.254) (layer F.Cu) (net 9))
 (segment (start 216.764 152.1051) (end 216.764 150.6908) (width 0.254) (layer F.Cu) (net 9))
 (segment (start 210.579 149.225) (end 211.8493 149.225) (width 0.254) (layer F.Cu) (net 9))
 (segment (start 212.1128 148.9615) (end 211.8493 149.225) (width 0.254) (layer F.Cu) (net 9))
 (segment (start 215.0347 148.9615) (end 212.1128 148.9615) (width 0.254) (layer F.Cu) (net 9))
 (segment (start 216.764 150.6908) (end 215.0347 148.9615) (width 0.254) (layer F.Cu) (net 9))
 (segment (start 216.764 152.1051) (end 216.764 153.5194) (width 0.254) (layer F.Cu) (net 9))
 (segment (start 217.3763 153.8368) (end 217.7418 153.4713) (width 0.254) (layer B.Cu) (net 9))
 (segment (start 217.3763 156.794) (end 217.3763 153.8368) (width 0.254) (layer B.Cu) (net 9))
 (segment (start 216.764 153.7587) (end 216.751 153.7717) (width 0.254) (layer F.Cu) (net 9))
 (segment (start 216.764 153.5194) (end 216.764 153.7587) (width 0.254) (layer F.Cu) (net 9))
 (segment (start 217.6937 153.5194) (end 216.764 153.5194) (width 0.254) (layer F.Cu) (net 9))
 (segment (start 217.7418 153.4713) (end 217.6937 153.5194) (width 0.254) (layer F.Cu) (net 9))
 (segment (start 215.722 156.794) (end 217.3763 156.794) (width 0.254) (layer B.Cu) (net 9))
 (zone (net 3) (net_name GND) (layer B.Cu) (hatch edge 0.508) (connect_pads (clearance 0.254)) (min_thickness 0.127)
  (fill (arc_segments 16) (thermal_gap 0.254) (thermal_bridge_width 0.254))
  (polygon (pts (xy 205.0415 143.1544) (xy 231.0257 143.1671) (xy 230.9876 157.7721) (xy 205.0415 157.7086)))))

